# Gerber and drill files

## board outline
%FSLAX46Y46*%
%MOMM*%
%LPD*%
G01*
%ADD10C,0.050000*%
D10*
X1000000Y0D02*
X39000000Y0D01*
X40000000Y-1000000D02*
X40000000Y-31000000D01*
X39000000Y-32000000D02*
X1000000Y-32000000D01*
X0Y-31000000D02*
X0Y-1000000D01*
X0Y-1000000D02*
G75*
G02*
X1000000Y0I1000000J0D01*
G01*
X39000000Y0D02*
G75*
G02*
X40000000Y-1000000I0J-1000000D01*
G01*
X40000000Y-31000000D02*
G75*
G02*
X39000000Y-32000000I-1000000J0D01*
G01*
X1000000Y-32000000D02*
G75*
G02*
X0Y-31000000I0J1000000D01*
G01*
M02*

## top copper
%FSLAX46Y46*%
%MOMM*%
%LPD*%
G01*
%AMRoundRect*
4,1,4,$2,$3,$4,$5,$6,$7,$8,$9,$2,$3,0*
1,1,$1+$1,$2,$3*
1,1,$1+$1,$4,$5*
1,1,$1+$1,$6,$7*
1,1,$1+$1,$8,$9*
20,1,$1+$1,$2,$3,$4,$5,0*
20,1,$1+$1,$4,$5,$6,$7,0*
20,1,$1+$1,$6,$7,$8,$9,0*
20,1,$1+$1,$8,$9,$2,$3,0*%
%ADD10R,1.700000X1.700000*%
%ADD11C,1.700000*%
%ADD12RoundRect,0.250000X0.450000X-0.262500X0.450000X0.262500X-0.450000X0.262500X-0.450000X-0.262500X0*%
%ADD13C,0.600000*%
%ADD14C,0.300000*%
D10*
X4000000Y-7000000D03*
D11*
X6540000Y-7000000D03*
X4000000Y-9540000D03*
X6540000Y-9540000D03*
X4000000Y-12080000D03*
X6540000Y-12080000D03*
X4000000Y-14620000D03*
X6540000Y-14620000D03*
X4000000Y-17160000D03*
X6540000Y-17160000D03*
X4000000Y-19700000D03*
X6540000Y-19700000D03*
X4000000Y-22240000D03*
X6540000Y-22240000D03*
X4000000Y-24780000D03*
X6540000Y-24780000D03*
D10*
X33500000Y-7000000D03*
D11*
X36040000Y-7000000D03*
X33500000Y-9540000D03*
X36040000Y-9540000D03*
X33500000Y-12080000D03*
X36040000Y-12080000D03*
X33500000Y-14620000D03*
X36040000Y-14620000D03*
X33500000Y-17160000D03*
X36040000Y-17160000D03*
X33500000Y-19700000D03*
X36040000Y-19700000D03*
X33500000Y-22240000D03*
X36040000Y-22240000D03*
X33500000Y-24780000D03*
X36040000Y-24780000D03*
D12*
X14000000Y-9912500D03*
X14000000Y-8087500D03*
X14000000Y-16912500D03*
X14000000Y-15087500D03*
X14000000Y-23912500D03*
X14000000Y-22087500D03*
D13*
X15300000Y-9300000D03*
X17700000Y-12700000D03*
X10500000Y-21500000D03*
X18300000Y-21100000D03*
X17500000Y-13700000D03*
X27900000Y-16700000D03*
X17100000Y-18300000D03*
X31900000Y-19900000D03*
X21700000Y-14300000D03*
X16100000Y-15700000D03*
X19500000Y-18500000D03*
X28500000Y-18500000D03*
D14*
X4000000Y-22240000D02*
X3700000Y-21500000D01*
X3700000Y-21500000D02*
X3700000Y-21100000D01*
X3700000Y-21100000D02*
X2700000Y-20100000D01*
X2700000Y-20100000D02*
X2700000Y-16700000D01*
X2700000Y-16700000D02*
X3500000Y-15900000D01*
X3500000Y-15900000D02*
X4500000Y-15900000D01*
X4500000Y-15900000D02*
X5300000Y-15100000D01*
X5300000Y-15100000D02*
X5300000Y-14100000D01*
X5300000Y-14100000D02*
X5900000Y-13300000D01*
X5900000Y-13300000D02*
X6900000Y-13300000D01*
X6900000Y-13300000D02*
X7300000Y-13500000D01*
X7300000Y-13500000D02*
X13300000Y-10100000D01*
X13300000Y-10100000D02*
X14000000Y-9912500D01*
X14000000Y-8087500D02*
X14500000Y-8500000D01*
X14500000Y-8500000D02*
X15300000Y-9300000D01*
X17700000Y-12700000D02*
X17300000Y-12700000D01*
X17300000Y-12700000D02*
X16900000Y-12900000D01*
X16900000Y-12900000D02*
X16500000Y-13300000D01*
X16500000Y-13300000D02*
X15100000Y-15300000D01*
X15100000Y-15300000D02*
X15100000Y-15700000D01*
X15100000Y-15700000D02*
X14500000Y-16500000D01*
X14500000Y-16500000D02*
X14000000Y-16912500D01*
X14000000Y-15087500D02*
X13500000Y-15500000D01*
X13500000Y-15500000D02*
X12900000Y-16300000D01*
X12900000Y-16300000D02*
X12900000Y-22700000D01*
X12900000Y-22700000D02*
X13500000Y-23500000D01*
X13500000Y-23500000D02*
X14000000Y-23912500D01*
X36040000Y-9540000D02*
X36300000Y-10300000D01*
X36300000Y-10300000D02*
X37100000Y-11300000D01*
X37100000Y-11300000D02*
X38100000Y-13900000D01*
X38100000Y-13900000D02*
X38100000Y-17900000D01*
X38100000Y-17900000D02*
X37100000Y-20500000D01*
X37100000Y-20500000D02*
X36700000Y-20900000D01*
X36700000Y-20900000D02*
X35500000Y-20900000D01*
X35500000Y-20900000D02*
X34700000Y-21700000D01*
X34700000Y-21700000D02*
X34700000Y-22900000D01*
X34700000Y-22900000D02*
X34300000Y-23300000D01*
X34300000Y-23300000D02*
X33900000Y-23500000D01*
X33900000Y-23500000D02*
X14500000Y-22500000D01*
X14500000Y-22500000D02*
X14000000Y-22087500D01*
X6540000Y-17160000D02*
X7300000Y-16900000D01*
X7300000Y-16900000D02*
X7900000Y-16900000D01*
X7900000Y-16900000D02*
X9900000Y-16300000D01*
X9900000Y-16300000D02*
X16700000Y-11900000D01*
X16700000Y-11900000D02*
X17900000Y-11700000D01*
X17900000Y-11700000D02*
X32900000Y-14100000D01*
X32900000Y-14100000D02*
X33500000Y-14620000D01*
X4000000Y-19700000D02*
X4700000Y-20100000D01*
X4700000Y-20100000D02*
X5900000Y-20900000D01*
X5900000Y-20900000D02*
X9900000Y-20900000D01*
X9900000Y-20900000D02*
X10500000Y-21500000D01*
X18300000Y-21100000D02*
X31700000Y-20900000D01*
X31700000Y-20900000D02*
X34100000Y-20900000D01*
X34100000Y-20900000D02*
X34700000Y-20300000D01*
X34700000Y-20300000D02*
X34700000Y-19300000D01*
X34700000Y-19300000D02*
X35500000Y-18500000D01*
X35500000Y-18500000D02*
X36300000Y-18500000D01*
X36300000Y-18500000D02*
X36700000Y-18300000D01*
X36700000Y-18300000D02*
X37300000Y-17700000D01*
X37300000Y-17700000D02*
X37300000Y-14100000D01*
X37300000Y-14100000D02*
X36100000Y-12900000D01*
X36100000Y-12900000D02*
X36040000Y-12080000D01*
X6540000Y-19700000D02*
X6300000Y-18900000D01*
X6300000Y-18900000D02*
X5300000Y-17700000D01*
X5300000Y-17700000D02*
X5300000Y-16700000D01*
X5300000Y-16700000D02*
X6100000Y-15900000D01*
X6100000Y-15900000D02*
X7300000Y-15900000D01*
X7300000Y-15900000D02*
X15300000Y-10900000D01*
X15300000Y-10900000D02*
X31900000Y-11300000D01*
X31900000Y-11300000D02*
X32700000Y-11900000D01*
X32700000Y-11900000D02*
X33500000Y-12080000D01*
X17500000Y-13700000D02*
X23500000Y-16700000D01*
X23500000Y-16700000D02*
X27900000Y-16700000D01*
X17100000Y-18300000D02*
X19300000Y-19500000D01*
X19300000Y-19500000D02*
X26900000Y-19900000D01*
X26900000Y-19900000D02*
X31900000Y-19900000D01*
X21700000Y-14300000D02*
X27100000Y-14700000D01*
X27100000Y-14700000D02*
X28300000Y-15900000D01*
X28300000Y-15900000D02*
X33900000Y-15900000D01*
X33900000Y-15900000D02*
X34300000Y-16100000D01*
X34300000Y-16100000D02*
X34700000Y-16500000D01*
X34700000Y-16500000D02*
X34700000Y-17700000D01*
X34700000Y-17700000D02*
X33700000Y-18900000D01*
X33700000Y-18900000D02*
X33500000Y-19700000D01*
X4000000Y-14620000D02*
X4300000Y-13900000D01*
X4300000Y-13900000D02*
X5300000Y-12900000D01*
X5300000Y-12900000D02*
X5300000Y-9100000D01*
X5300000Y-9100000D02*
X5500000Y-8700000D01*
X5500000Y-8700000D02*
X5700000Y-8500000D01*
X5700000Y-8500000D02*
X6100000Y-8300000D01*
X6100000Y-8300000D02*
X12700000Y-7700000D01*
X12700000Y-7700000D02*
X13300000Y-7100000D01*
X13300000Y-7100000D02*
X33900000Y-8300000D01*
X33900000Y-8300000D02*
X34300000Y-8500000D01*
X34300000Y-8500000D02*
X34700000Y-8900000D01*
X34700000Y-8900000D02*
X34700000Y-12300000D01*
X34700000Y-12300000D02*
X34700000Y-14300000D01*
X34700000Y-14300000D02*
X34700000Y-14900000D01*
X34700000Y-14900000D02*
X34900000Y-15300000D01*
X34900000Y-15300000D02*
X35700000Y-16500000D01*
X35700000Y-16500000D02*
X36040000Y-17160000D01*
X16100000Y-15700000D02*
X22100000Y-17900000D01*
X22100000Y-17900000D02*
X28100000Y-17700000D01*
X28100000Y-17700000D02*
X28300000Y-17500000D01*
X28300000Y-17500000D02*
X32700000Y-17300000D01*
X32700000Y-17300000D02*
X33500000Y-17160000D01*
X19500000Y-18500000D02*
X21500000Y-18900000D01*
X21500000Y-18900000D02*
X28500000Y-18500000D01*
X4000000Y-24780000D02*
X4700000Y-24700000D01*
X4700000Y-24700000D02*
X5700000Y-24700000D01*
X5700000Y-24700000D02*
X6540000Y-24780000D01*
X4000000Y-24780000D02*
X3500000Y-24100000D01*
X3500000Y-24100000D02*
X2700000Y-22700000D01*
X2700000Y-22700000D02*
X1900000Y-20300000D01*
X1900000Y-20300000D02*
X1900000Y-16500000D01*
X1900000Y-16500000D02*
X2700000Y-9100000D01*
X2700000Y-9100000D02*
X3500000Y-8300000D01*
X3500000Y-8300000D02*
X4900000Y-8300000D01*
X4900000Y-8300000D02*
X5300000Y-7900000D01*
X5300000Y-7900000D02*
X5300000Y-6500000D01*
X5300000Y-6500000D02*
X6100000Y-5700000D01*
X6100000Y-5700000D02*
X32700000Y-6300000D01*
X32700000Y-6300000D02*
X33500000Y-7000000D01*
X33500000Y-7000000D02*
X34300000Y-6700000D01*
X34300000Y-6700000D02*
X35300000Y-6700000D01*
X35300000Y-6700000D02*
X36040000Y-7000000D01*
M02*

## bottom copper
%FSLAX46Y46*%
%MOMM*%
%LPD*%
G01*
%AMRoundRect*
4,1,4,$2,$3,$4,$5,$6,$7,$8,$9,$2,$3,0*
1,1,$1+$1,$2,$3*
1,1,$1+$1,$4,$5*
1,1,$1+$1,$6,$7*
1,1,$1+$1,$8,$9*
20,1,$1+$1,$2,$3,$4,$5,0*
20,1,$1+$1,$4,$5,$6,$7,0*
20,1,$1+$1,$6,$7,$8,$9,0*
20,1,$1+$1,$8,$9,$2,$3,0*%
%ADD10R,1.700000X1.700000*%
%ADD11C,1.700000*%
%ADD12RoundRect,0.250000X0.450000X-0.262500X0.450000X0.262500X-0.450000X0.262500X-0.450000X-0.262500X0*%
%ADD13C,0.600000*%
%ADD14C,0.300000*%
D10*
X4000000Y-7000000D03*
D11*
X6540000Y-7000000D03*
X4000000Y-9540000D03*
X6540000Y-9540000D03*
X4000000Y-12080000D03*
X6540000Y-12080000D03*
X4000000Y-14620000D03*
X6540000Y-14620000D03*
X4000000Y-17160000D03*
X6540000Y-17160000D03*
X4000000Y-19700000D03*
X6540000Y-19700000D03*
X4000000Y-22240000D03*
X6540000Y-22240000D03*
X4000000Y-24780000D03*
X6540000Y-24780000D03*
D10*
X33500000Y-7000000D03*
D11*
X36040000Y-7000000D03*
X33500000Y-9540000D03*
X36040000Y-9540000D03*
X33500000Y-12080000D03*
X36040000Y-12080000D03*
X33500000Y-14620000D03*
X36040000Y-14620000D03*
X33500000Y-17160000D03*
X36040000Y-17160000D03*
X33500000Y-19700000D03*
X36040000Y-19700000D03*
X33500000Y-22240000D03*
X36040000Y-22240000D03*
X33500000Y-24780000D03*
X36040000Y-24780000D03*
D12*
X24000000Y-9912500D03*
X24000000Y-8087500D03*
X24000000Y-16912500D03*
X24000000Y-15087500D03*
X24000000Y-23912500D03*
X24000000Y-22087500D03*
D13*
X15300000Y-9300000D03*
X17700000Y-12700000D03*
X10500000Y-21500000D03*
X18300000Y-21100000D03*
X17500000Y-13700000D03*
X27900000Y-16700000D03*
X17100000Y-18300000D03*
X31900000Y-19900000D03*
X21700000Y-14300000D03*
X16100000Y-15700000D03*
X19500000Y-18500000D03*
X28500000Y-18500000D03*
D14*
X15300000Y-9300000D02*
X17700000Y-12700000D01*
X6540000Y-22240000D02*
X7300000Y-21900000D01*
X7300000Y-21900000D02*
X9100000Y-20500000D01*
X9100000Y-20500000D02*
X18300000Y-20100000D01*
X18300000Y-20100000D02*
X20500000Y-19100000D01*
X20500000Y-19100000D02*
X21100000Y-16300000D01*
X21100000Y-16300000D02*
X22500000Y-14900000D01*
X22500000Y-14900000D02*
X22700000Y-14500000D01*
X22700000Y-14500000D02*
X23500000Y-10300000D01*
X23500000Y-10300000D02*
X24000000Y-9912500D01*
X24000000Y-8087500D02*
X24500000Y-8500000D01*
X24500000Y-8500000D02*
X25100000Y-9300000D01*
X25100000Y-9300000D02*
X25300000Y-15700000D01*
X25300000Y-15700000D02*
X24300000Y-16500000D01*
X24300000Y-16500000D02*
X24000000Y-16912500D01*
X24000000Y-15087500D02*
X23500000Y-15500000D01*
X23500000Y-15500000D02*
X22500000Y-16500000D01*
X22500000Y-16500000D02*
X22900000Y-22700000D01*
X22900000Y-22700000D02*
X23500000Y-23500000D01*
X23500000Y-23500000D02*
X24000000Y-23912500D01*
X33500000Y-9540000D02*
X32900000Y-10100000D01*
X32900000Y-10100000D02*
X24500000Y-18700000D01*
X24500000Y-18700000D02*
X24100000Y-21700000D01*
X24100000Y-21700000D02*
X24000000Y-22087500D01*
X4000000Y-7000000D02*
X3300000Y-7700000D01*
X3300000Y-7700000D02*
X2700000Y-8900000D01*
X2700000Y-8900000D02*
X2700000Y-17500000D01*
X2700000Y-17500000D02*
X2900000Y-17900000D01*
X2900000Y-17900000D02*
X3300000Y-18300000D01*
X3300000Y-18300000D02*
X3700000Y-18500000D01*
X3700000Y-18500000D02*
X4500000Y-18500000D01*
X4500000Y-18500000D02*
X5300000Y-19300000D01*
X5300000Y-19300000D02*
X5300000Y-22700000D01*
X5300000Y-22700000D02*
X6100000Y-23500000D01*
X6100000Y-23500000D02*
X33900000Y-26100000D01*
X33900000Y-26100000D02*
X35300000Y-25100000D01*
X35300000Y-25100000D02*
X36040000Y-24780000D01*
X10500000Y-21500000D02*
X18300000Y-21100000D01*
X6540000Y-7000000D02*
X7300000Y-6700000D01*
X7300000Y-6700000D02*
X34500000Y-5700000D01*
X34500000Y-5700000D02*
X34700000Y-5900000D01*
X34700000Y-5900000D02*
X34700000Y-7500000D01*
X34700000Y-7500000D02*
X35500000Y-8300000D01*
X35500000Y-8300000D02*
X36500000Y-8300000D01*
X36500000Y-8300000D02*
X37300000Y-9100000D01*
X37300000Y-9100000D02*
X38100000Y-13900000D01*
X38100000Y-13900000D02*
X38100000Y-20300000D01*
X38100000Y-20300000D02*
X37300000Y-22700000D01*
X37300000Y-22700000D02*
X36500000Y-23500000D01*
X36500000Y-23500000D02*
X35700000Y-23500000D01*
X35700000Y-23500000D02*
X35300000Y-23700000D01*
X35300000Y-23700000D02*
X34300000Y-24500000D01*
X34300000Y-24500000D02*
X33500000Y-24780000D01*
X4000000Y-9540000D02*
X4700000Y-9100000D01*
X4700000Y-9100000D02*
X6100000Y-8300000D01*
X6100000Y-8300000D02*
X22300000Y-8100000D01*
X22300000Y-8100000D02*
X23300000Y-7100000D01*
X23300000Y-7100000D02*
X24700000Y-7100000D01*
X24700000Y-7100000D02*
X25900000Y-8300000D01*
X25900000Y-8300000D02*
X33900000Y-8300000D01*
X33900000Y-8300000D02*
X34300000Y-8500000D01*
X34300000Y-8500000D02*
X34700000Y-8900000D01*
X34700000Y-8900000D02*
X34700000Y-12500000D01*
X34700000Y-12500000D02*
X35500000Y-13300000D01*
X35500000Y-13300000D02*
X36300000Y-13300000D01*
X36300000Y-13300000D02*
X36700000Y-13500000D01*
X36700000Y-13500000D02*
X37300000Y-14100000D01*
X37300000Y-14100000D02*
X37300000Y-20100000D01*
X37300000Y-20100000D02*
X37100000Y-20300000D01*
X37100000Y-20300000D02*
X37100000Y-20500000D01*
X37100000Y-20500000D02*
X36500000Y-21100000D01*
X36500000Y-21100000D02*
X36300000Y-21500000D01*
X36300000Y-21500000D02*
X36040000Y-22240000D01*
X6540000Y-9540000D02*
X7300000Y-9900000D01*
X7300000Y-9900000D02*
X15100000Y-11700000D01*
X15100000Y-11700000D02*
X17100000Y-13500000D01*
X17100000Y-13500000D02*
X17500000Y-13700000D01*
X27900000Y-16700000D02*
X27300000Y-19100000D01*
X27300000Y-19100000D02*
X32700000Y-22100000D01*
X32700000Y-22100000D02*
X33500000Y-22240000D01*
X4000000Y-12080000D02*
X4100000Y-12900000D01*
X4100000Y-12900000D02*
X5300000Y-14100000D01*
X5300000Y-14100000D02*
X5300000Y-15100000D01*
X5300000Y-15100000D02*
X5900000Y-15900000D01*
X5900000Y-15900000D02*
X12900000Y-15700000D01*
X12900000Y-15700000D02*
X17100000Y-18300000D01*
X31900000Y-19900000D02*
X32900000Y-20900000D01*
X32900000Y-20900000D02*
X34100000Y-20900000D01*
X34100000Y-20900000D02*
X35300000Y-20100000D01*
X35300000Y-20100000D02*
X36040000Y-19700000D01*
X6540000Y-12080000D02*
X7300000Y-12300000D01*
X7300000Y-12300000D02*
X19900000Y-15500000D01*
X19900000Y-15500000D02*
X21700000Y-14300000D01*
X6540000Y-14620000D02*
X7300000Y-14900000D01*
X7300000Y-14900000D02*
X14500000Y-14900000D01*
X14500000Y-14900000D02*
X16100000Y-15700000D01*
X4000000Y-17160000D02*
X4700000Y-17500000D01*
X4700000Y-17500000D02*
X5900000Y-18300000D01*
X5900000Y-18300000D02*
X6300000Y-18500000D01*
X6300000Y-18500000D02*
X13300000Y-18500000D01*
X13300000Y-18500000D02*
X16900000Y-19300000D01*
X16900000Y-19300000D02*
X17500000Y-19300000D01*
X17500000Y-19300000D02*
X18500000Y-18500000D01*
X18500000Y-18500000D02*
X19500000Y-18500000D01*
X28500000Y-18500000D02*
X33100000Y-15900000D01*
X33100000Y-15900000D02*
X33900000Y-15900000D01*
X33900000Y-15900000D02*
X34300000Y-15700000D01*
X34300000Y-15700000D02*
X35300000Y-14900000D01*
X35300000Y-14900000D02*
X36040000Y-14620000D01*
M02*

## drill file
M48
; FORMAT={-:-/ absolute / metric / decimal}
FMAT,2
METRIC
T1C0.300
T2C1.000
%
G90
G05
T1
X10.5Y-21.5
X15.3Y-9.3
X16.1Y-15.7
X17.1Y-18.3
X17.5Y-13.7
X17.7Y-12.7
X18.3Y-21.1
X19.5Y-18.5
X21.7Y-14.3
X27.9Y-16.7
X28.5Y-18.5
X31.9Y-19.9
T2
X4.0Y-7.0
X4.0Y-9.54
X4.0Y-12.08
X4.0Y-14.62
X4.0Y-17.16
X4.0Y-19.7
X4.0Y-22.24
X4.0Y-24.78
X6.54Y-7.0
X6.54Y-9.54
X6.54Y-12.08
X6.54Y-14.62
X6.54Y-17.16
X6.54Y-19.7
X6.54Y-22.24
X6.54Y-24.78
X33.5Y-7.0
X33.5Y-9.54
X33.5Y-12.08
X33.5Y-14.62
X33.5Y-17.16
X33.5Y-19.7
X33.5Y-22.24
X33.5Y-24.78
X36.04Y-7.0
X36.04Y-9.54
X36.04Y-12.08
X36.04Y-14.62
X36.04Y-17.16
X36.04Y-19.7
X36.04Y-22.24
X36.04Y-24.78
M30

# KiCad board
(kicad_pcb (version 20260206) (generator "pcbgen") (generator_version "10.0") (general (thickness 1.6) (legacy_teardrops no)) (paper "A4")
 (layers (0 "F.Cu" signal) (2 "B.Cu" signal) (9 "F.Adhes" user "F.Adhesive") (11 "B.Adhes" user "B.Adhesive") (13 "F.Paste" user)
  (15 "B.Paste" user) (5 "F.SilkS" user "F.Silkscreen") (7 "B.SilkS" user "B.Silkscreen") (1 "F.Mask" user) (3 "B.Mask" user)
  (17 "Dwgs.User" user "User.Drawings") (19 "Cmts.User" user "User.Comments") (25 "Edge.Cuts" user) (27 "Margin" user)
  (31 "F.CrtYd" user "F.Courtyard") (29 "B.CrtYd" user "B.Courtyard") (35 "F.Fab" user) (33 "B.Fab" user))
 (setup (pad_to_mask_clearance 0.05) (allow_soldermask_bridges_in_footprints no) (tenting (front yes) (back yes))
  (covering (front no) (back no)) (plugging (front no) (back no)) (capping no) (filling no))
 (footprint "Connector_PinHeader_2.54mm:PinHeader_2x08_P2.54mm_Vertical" (layer "F.Cu") (at 4 7)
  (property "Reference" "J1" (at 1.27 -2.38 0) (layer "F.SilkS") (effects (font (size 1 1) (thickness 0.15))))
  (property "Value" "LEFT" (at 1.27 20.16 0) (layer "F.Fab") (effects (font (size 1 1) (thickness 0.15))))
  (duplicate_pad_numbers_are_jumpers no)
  (pad "1" thru_hole rect (at 0 0) (size 1.7 1.7) (drill 1) (layers "*.Cu" "*.Mask") (remove_unused_layers no) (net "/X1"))
  (pad "2" thru_hole circle (at 2.54 0) (size 1.7 1.7) (drill 1) (layers "*.Cu" "*.Mask") (remove_unused_layers no) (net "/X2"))
  (pad "3" thru_hole circle (at 0 2.54) (size 1.7 1.7) (drill 1) (layers "*.Cu" "*.Mask") (remove_unused_layers no) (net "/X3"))
  (pad "4" thru_hole circle (at 2.54 2.54) (size 1.7 1.7) (drill 1) (layers "*.Cu" "*.Mask") (remove_unused_layers no) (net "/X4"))
  (pad "5" thru_hole circle (at 0 5.08) (size 1.7 1.7) (drill 1) (layers "*.Cu" "*.Mask") (remove_unused_layers no) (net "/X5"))
  (pad "6" thru_hole circle (at 2.54 5.08) (size 1.7 1.7) (drill 1) (layers "*.Cu" "*.Mask") (remove_unused_layers no) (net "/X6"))
  (pad "7" thru_hole circle (at 0 7.62) (size 1.7 1.7) (drill 1) (layers "*.Cu" "*.Mask") (remove_unused_layers no) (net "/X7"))
  (pad "8" thru_hole circle (at 2.54 7.62) (size 1.7 1.7) (drill 1) (layers "*.Cu" "*.Mask") (remove_unused_layers no) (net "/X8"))
  (pad "9" thru_hole circle (at 0 10.16) (size 1.7 1.7) (drill 1) (layers "*.Cu" "*.Mask") (remove_unused_layers no) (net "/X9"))
  (pad "10" thru_hole circle (at 2.54 10.16) (size 1.7 1.7) (drill 1) (layers "*.Cu" "*.Mask") (remove_unused_layers no) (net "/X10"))
  (pad "11" thru_hole circle (at 0 12.7) (size 1.7 1.7) (drill 1) (layers "*.Cu" "*.Mask") (remove_unused_layers no) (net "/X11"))
  (pad "12" thru_hole circle (at 2.54 12.7) (size 1.7 1.7) (drill 1) (layers "*.Cu" "*.Mask") (remove_unused_layers no) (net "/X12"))
  (pad "13" thru_hole circle (at 0 15.24) (size 1.7 1.7) (drill 1) (layers "*.Cu" "*.Mask") (remove_unused_layers no) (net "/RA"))
  (pad "14" thru_hole circle (at 2.54 15.24) (size 1.7 1.7) (drill 1) (layers "*.Cu" "*.Mask") (remove_unused_layers no) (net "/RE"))
  (pad "15" thru_hole circle (at 0 17.78) (size 1.7 1.7) (drill 1) (layers "*.Cu" "*.Mask") (remove_unused_layers no) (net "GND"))
  (pad "16" thru_hole circle (at 2.54 17.78) (size 1.7 1.7) (drill 1) (layers "*.Cu" "*.Mask") (remove_unused_layers no) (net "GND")))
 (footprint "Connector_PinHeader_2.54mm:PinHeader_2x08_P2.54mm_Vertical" (layer "F.Cu") (at 33.5 7)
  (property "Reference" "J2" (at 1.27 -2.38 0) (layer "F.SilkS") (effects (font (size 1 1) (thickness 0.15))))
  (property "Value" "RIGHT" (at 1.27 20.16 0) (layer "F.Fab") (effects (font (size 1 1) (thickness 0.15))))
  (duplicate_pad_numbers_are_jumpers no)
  (pad "1" thru_hole rect (at 0 0) (size 1.7 1.7) (drill 1) (layers "*.Cu" "*.Mask") (remove_unused_layers no) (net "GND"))
  (pad "2" thru_hole circle (at 2.54 0) (size 1.7 1.7) (drill 1) (layers "*.Cu" "*.Mask") (remove_unused_layers no) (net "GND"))
  (pad "3" thru_hole circle (at 0 2.54) (size 1.7 1.7) (drill 1) (layers "*.Cu" "*.Mask") (remove_unused_layers no) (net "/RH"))
  (pad "4" thru_hole circle (at 2.54 2.54) (size 1.7 1.7) (drill 1) (layers "*.Cu" "*.Mask") (remove_unused_layers no) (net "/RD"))
  (pad "5" thru_hole circle (at 0 5.08) (size 1.7 1.7) (drill 1) (layers "*.Cu" "*.Mask") (remove_unused_layers no) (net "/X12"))
  (pad "6" thru_hole circle (at 2.54 5.08) (size 1.7 1.7) (drill 1) (layers "*.Cu" "*.Mask") (remove_unused_layers no) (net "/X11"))
  (pad "7" thru_hole circle (at 0 7.62) (size 1.7 1.7) (drill 1) (layers "*.Cu" "*.Mask") (remove_unused_layers no) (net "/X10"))
  (pad "8" thru_hole circle (at 2.54 7.62) (size 1.7 1.7) (drill 1) (layers "*.Cu" "*.Mask") (remove_unused_layers no) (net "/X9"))
  (pad "9" thru_hole circle (at 0 10.16) (size 1.7 1.7) (drill 1) (layers "*.Cu" "*.Mask") (remove_unused_layers no) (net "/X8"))
  (pad "10" thru_hole circle (at 2.54 10.16) (size 1.7 1.7) (drill 1) (layers "*.Cu" "*.Mask") (remove_unused_layers no) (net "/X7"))
  (pad "11" thru_hole circle (at 0 12.7) (size 1.7 1.7) (drill 1) (layers "*.Cu" "*.Mask") (remove_unused_layers no) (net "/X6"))
  (pad "12" thru_hole circle (at 2.54 12.7) (size 1.7 1.7) (drill 1) (layers "*.Cu" "*.Mask") (remove_unused_layers no) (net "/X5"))
  (pad "13" thru_hole circle (at 0 15.24) (size 1.7 1.7) (drill 1) (layers "*.Cu" "*.Mask") (remove_unused_layers no) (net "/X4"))
  (pad "14" thru_hole circle (at 2.54 15.24) (size 1.7 1.7) (drill 1) (layers "*.Cu" "*.Mask") (remove_unused_layers no) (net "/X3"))
  (pad "15" thru_hole circle (at 0 17.78) (size 1.7 1.7) (drill 1) (layers "*.Cu" "*.Mask") (remove_unused_layers no) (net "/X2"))
  (pad "16" thru_hole circle (at 2.54 17.78) (size 1.7 1.7) (drill 1) (layers "*.Cu" "*.Mask") (remove_unused_layers no) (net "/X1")))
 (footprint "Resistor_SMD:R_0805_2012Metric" (layer "F.Cu") (at 14 9 90)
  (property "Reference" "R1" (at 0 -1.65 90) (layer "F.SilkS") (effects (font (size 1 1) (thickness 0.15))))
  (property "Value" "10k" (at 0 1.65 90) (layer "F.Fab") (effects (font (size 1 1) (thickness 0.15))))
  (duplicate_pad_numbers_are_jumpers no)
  (pad "1" smd roundrect (at -0.9125 0 90) (size 1.025 1.4) (layers "F.Cu" "F.Mask" "F.Paste") (roundrect_rratio 0.243902) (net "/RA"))
  (pad "2" smd roundrect (at 0.9125 0 90) (size 1.025 1.4) (layers "F.Cu" "F.Mask" "F.Paste") (roundrect_rratio 0.243902) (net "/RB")))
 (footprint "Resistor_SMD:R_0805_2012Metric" (layer "F.Cu") (at 14 16 90)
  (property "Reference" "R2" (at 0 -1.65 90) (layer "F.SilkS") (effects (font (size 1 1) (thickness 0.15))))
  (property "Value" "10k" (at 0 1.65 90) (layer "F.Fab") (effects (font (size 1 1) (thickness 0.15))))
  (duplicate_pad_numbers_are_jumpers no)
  (pad "1" smd roundrect (at -0.9125 0 90) (size 1.025 1.4) (layers "F.Cu" "F.Mask" "F.Paste") (roundrect_rratio 0.243902) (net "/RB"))
  (pad "2" smd roundrect (at 0.9125 0 90) (size 1.025 1.4) (layers "F.Cu" "F.Mask" "F.Paste") (roundrect_rratio 0.243902) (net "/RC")))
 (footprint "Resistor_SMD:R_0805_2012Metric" (layer "F.Cu") (at 14 23 90)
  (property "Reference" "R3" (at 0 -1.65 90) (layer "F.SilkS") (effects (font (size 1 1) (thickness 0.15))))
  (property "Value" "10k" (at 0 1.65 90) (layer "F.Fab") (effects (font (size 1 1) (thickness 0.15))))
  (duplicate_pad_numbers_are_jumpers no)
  (pad "1" smd roundrect (at -0.9125 0 90) (size 1.025 1.4) (layers "F.Cu" "F.Mask" "F.Paste") (roundrect_rratio 0.243902) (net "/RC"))
  (pad "2" smd roundrect (at 0.9125 0 90) (size 1.025 1.4) (layers "F.Cu" "F.Mask" "F.Paste") (roundrect_rratio 0.243902) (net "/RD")))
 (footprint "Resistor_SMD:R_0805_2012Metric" (layer "B.Cu") (at 24 9 90)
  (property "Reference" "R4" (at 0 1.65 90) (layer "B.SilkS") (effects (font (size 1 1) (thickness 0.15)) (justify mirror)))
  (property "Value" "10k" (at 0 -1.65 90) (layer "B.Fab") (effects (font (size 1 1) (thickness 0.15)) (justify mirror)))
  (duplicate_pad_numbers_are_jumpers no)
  (pad "1" smd roundrect (at -0.9125 0 90) (size 1.025 1.4) (layers "B.Cu" "B.Mask" "B.Paste") (roundrect_rratio 0.243902) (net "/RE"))
  (pad "2" smd roundrect (at 0.9125 0 90) (size 1.025 1.4) (layers "B.Cu" "B.Mask" "B.Paste") (roundrect_rratio 0.243902) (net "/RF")))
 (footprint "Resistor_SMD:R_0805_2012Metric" (layer "B.Cu") (at 24 16 90)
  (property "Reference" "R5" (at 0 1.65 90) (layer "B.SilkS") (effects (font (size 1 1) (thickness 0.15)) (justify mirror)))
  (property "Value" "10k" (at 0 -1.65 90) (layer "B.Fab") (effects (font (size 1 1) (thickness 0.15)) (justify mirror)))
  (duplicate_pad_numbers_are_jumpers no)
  (pad "1" smd roundrect (at -0.9125 0 90) (size 1.025 1.4) (layers "B.Cu" "B.Mask" "B.Paste") (roundrect_rratio 0.243902) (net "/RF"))
  (pad "2" smd roundrect (at 0.9125 0 90) (size 1.025 1.4) (layers "B.Cu" "B.Mask" "B.Paste") (roundrect_rratio 0.243902) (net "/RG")))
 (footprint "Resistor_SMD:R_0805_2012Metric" (layer "B.Cu") (at 24 23 90)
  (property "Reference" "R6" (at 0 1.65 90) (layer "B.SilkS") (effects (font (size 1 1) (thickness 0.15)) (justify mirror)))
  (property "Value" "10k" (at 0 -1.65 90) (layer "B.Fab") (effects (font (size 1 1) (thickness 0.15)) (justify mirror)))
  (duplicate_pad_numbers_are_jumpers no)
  (pad "1" smd roundrect (at -0.9125 0 90) (size 1.025 1.4) (layers "B.Cu" "B.Mask" "B.Paste") (roundrect_rratio 0.243902) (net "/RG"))
  (pad "2" smd roundrect (at 0.9125 0 90) (size 1.025 1.4) (layers "B.Cu" "B.Mask" "B.Paste") (roundrect_rratio 0.243902) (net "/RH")))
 (gr_line (start 1 0) (end 39 0) (stroke (width 0.05) (type default)) (layer "Edge.Cuts"))
 (gr_line (start 40 1) (end 40 31) (stroke (width 0.05) (type default)) (layer "Edge.Cuts"))
 (gr_line (start 39 32) (end 1 32) (stroke (width 0.05) (type default)) (layer "Edge.Cuts"))
 (gr_line (start 0 31) (end 0 1) (stroke (width 0.05) (type default)) (layer "Edge.Cuts"))
 (gr_arc (start 0 1) (mid 0.292893 0.292893) (end 1 0) (stroke (width 0.05) (type default)) (layer "Edge.Cuts"))
 (gr_arc (start 39 0) (mid 39.707107 0.292893) (end 40 1) (stroke (width 0.05) (type default)) (layer "Edge.Cuts"))
 (gr_arc (start 40 31) (mid 39.707107 31.707107) (end 39 32) (stroke (width 0.05) (type default)) (layer "Edge.Cuts"))
 (gr_arc (start 1 32) (mid 0.292893 31.707107) (end 0 31) (stroke (width 0.05) (type default)) (layer "Edge.Cuts"))
 (segment (start 4 22.24) (end 3.7 21.5) (width 0.3) (layer "F.Cu") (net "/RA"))
 (segment (start 3.7 21.5) (end 3.7 21.1) (width 0.3) (layer "F.Cu") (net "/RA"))
 (segment (start 3.7 21.1) (end 2.7 20.1) (width 0.3) (layer "F.Cu") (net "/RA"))
 (segment (start 2.7 20.1) (end 2.7 16.7) (width 0.3) (layer "F.Cu") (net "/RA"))
 (segment (start 2.7 16.7) (end 3.5 15.9) (width 0.3) (layer "F.Cu") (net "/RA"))
 (segment (start 3.5 15.9) (end 4.5 15.9) (width 0.3) (layer "F.Cu") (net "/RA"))
 (segment (start 4.5 15.9) (end 5.3 15.1) (width 0.3) (layer "F.Cu") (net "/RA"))
 (segment (start 5.3 15.1) (end 5.3 14.1) (width 0.3) (layer "F.Cu") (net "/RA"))
 (segment (start 5.3 14.1) (end 5.9 13.3) (width 0.3) (layer "F.Cu") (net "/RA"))
 (segment (start 5.9 13.3) (end 6.9 13.3) (width 0.3) (layer "F.Cu") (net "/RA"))
 (segment (start 6.9 13.3) (end 7.3 13.5) (width 0.3) (layer "F.Cu") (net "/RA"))
 (segment (start 7.3 13.5) (end 13.3 10.1) (width 0.3) (layer "F.Cu") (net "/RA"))
 (segment (start 13.3 10.1) (end 14 9.9125) (width 0.3) (layer "F.Cu") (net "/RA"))
 (segment (start 14 8.0875) (end 14.5 8.5) (width 0.3) (layer "F.Cu") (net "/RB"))
 (segment (start 14.5 8.5) (end 15.3 9.3) (width 0.3) (layer "F.Cu") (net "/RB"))
 (segment (start 15.3 9.3) (end 17.7 12.7) (width 0.3) (layer "B.Cu") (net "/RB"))
 (segment (start 17.7 12.7) (end 17.3 12.7) (width 0.3) (layer "F.Cu") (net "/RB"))
 (segment (start 17.3 12.7) (end 16.9 12.9) (width 0.3) (layer "F.Cu") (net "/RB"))
 (segment (start 16.9 12.9) (end 16.5 13.3) (width 0.3) (layer "F.Cu") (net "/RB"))
 (segment (start 16.5 13.3) (end 15.1 15.3) (width 0.3) (layer "F.Cu") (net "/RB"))
 (segment (start 15.1 15.3) (end 15.1 15.7) (width 0.3) (layer "F.Cu") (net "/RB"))
 (segment (start 15.1 15.7) (end 14.5 16.5) (width 0.3) (layer "F.Cu") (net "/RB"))
 (segment (start 14.5 16.5) (end 14 16.9125) (width 0.3) (layer "F.Cu") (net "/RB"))
 (segment (start 14 15.0875) (end 13.5 15.5) (width 0.3) (layer "F.Cu") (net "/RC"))
 (segment (start 13.5 15.5) (end 12.9 16.3) (width 0.3) (layer "F.Cu") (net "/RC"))
 (segment (start 12.9 16.3) (end 12.9 22.7) (width 0.3) (layer "F.Cu") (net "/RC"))
 (segment (start 12.9 22.7) (end 13.5 23.5) (width 0.3) (layer "F.Cu") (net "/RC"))
 (segment (start 13.5 23.5) (end 14 23.9125) (width 0.3) (layer "F.Cu") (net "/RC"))
 (segment (start 36.04 9.54) (end 36.3 10.3) (width 0.3) (layer "F.Cu") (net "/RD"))
 (segment (start 36.3 10.3) (end 37.1 11.3) (width 0.3) (layer "F.Cu") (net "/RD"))
 (segment (start 37.1 11.3) (end 38.1 13.9) (width 0.3) (layer "F.Cu") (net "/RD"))
 (segment (start 38.1 13.9) (end 38.1 17.9) (width 0.3) (layer "F.Cu") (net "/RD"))
 (segment (start 38.1 17.9) (end 37.1 20.5) (width 0.3) (layer "F.Cu") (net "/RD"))
 (segment (start 37.1 20.5) (end 36.7 20.9) (width 0.3) (layer "F.Cu") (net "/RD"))
 (segment (start 36.7 20.9) (end 35.5 20.9) (width 0.3) (layer "F.Cu") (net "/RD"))
 (segment (start 35.5 20.9) (end 34.7 21.7) (width 0.3) (layer "F.Cu") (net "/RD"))
 (segment (start 34.7 21.7) (end 34.7 22.9) (width 0.3) (layer "F.Cu") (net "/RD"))
 (segment (start 34.7 22.9) (end 34.3 23.3) (width 0.3) (layer "F.Cu") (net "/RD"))
 (segment (start 34.3 23.3) (end 33.9 23.5) (width 0.3) (layer "F.Cu") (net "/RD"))
 (segment (start 33.9 23.5) (end 14.5 22.5) (width 0.3) (layer "F.Cu") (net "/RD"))
 (segment (start 14.5 22.5) (end 14 22.0875) (width 0.3) (layer "F.Cu") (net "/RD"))
 (segment (start 6.54 22.24) (end 7.3 21.9) (width 0.3) (layer "B.Cu") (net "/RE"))
 (segment (start 7.3 21.9) (end 9.1 20.5) (width 0.3) (layer "B.Cu") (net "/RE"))
 (segment (start 9.1 20.5) (end 18.3 20.1) (width 0.3) (layer "B.Cu") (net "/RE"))
 (segment (start 18.3 20.1) (end 20.5 19.1) (width 0.3) (layer "B.Cu") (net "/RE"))
 (segment (start 20.5 19.1) (end 21.1 16.3) (width 0.3) (layer "B.Cu") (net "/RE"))
 (segment (start 21.1 16.3) (end 22.5 14.9) (width 0.3) (layer "B.Cu") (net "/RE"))
 (segment (start 22.5 14.9) (end 22.7 14.5) (width 0.3) (layer "B.Cu") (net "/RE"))
 (segment (start 22.7 14.5) (end 23.5 10.3) (width 0.3) (layer "B.Cu") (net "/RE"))
 (segment (start 23.5 10.3) (end 24 9.9125) (width 0.3) (layer "B.Cu") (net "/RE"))
 (segment (start 24 8.0875) (end 24.5 8.5) (width 0.3) (layer "B.Cu") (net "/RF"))
 (segment (start 24.5 8.5) (end 25.1 9.3) (width 0.3) (layer "B.Cu") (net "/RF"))
 (segment (start 25.1 9.3) (end 25.3 15.7) (width 0.3) (layer "B.Cu") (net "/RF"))
 (segment (start 25.3 15.7) (end 24.3 16.5) (width 0.3) (layer "B.Cu") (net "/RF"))
 (segment (start 24.3 16.5) (end 24 16.9125) (width 0.3) (layer "B.Cu") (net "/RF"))
 (segment (start 24 15.0875) (end 23.5 15.5) (width 0.3) (layer "B.Cu") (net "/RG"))
 (segment (start 23.5 15.5) (end 22.5 16.5) (width 0.3) (layer "B.Cu") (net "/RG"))
 (segment (start 22.5 16.5) (end 22.9 22.7) (width 0.3) (layer "B.Cu") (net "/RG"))
 (segment (start 22.9 22.7) (end 23.5 23.5) (width 0.3) (layer "B.Cu") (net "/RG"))
 (segment (start 23.5 23.5) (end 24 23.9125) (width 0.3) (layer "B.Cu") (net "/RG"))
 (segment (start 33.5 9.54) (end 32.9 10.1) (width 0.3) (layer "B.Cu") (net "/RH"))
 (segment (start 32.9 10.1) (end 24.5 18.7) (width 0.3) (layer "B.Cu") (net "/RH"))
 (segment (start 24.5 18.7) (end 24.1 21.7) (width 0.3) (layer "B.Cu") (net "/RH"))
 (segment (start 24.1 21.7) (end 24 22.0875) (width 0.3) (layer "B.Cu") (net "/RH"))
 (segment (start 4 7) (end 3.3 7.7) (width 0.3) (layer "B.Cu") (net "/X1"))
 (segment (start 3.3 7.7) (end 2.7 8.9) (width 0.3) (layer "B.Cu") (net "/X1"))
 (segment (start 2.7 8.9) (end 2.7 17.5) (width 0.3) (layer "B.Cu") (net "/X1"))
 (segment (start 2.7 17.5) (end 2.9 17.9) (width 0.3) (layer "B.Cu") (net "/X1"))
 (segment (start 2.9 17.9) (end 3.3 18.3) (width 0.3) (layer "B.Cu") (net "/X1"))
 (segment (start 3.3 18.3) (end 3.7 18.5) (width 0.3) (layer "B.Cu") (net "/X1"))
 (segment (start 3.7 18.5) (end 4.5 18.5) (width 0.3) (layer "B.Cu") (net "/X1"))
 (segment (start 4.5 18.5) (end 5.3 19.3) (width 0.3) (layer "B.Cu") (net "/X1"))
 (segment (start 5.3 19.3) (end 5.3 22.7) (width 0.3) (layer "B.Cu") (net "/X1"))
 (segment (start 5.3 22.7) (end 6.1 23.5) (width 0.3) (layer "B.Cu") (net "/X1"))
 (segment (start 6.1 23.5) (end 33.9 26.1) (width 0.3) (layer "B.Cu") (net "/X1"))
 (segment (start 33.9 26.1) (end 35.3 25.1) (width 0.3) (layer "B.Cu") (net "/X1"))
 (segment (start 35.3 25.1) (end 36.04 24.78) (width 0.3) (layer "B.Cu") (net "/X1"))
 (segment (start 6.54 17.16) (end 7.3 16.9) (width 0.3) (layer "F.Cu") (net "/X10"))
 (segment (start 7.3 16.9) (end 7.9 16.9) (width 0.3) (layer "F.Cu") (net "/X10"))
 (segment (start 7.9 16.9) (end 9.9 16.3) (width 0.3) (layer "F.Cu") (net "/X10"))
 (segment (start 9.9 16.3) (end 16.7 11.9) (width 0.3) (layer "F.Cu") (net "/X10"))
 (segment (start 16.7 11.9) (end 17.9 11.7) (width 0.3) (layer "F.Cu") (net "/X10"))
 (segment (start 17.9 11.7) (end 32.9 14.1) (width 0.3) (layer "F.Cu") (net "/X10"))
 (segment (start 32.9 14.1) (end 33.5 14.62) (width 0.3) (layer "F.Cu") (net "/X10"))
 (segment (start 4 19.7) (end 4.7 20.1) (width 0.3) (layer "F.Cu") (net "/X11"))
 (segment (start 4.7 20.1) (end 5.9 20.9) (width 0.3) (layer "F.Cu") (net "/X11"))
 (segment (start 5.9 20.9) (end 9.9 20.9) (width 0.3) (layer "F.Cu") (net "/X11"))
 (segment (start 9.9 20.9) (end 10.5 21.5) (width 0.3) (layer "F.Cu") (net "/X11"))
 (segment (start 10.5 21.5) (end 18.3 21.1) (width 0.3) (layer "B.Cu") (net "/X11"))
 (segment (start 18.3 21.1) (end 31.7 20.9) (width 0.3) (layer "F.Cu") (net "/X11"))
 (segment (start 31.7 20.9) (end 34.1 20.9) (width 0.3) (layer "F.Cu") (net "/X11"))
 (segment (start 34.1 20.9) (end 34.7 20.3) (width 0.3) (layer "F.Cu") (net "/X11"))
 (segment (start 34.7 20.3) (end 34.7 19.3) (width 0.3) (layer "F.Cu") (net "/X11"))
 (segment (start 34.7 19.3) (end 35.5 18.5) (width 0.3) (layer "F.Cu") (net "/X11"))
 (segment (start 35.5 18.5) (end 36.3 18.5) (width 0.3) (layer "F.Cu") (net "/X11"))
 (segment (start 36.3 18.5) (end 36.7 18.3) (width 0.3) (layer "F.Cu") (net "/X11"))
 (segment (start 36.7 18.3) (end 37.3 17.7) (width 0.3) (layer "F.Cu") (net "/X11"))
 (segment (start 37.3 17.7) (end 37.3 14.1) (width 0.3) (layer "F.Cu") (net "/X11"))
 (segment (start 37.3 14.1) (end 36.1 12.9) (width 0.3) (layer "F.Cu") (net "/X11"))
 (segment (start 36.1 12.9) (end 36.04 12.08) (width 0.3) (layer "F.Cu") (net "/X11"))
 (segment (start 6.54 19.7) (end 6.3 18.9) (width 0.3) (layer "F.Cu") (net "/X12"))
 (segment (start 6.3 18.9) (end 5.3 17.7) (width 0.3) (layer "F.Cu") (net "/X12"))
 (segment (start 5.3 17.7) (end 5.3 16.7) (width 0.3) (layer "F.Cu") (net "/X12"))
 (segment (start 5.3 16.7) (end 6.1 15.9) (width 0.3) (layer "F.Cu") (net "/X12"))
 (segment (start 6.1 15.9) (end 7.3 15.9) (width 0.3) (layer "F.Cu") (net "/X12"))
 (segment (start 7.3 15.9) (end 15.3 10.9) (width 0.3) (layer "F.Cu") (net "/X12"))
 (segment (start 15.3 10.9) (end 31.9 11.3) (width 0.3) (layer "F.Cu") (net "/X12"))
 (segment (start 31.9 11.3) (end 32.7 11.9) (width 0.3) (layer "F.Cu") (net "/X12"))
 (segment (start 32.7 11.9) (end 33.5 12.08) (width 0.3) (layer "F.Cu") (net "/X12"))
 (segment (start 6.54 7) (end 7.3 6.7) (width 0.3) (layer "B.Cu") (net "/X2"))
 (segment (start 7.3 6.7) (end 34.5 5.7) (width 0.3) (layer "B.Cu") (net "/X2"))
 (segment (start 34.5 5.7) (end 34.7 5.9) (width 0.3) (layer "B.Cu") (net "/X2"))
 (segment (start 34.7 5.9) (end 34.7 7.5) (width 0.3) (layer "B.Cu") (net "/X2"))
 (segment (start 34.7 7.5) (end 35.5 8.3) (width 0.3) (layer "B.Cu") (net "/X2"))
 (segment (start 35.5 8.3) (end 36.5 8.3) (width 0.3) (layer "B.Cu") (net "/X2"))
 (segment (start 36.5 8.3) (end 37.3 9.1) (width 0.3) (layer "B.Cu") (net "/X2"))
 (segment (start 37.3 9.1) (end 38.1 13.9) (width 0.3) (layer "B.Cu") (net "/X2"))
 (segment (start 38.1 13.9) (end 38.1 20.3) (width 0.3) (layer "B.Cu") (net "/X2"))
 (segment (start 38.1 20.3) (end 37.3 22.7) (width 0.3) (layer "B.Cu") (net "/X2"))
 (segment (start 37.3 22.7) (end 36.5 23.5) (width 0.3) (layer "B.Cu") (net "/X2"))
 (segment (start 36.5 23.5) (end 35.7 23.5) (width 0.3) (layer "B.Cu") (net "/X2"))
 (segment (start 35.7 23.5) (end 35.3 23.7) (width 0.3) (layer "B.Cu") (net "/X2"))
 (segment (start 35.3 23.7) (end 34.3 24.5) (width 0.3) (layer "B.Cu") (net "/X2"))
 (segment (start 34.3 24.5) (end 33.5 24.78) (width 0.3) (layer "B.Cu") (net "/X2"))
 (segment (start 4 9.54) (end 4.7 9.1) (width 0.3) (layer "B.Cu") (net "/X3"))
 (segment (start 4.7 9.1) (end 6.1 8.3) (width 0.3) (layer "B.Cu") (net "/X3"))
 (segment (start 6.1 8.3) (end 22.3 8.1) (width 0.3) (layer "B.Cu") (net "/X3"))
 (segment (start 22.3 8.1) (end 23.3 7.1) (width 0.3) (layer "B.Cu") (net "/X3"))
 (segment (start 23.3 7.1) (end 24.7 7.1) (width 0.3) (layer "B.Cu") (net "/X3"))
 (segment (start 24.7 7.1) (end 25.9 8.3) (width 0.3) (layer "B.Cu") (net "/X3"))
 (segment (start 25.9 8.3) (end 33.9 8.3) (width 0.3) (layer "B.Cu") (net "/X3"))
 (segment (start 33.9 8.3) (end 34.3 8.5) (width 0.3) (layer "B.Cu") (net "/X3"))
 (segment (start 34.3 8.5) (end 34.7 8.9) (width 0.3) (layer "B.Cu") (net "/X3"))
 (segment (start 34.7 8.9) (end 34.7 12.5) (width 0.3) (layer "B.Cu") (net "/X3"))
 (segment (start 34.7 12.5) (end 35.5 13.3) (width 0.3) (layer "B.Cu") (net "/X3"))
 (segment (start 35.5 13.3) (end 36.3 13.3) (width 0.3) (layer "B.Cu") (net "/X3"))
 (segment (start 36.3 13.3) (end 36.7 13.5) (width 0.3) (layer "B.Cu") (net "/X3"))
 (segment (start 36.7 13.5) (end 37.3 14.1) (width 0.3) (layer "B.Cu") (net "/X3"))
 (segment (start 37.3 14.1) (end 37.3 20.1) (width 0.3) (layer "B.Cu") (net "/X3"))
 (segment (start 37.3 20.1) (end 37.1 20.3) (width 0.3) (layer "B.Cu") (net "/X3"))
 (segment (start 37.1 20.3) (end 37.1 20.5) (width 0.3) (layer "B.Cu") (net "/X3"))
 (segment (start 37.1 20.5) (end 36.5 21.1) (width 0.3) (layer "B.Cu") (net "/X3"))
 (segment (start 36.5 21.1) (end 36.3 21.5) (width 0.3) (layer "B.Cu") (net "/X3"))
 (segment (start 36.3 21.5) (end 36.04 22.24) (width 0.3) (layer "B.Cu") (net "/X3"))
 (segment (start 6.54 9.54) (end 7.3 9.9) (width 0.3) (layer "B.Cu") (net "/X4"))
 (segment (start 7.3 9.9) (end 15.1 11.7) (width 0.3) (layer "B.Cu") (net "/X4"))
 (segment (start 15.1 11.7) (end 17.1 13.5) (width 0.3) (layer "B.Cu") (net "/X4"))
 (segment (start 17.1 13.5) (end 17.5 13.7) (width 0.3) (layer "B.Cu") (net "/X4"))
 (segment (start 17.5 13.7) (end 23.5 16.7) (width 0.3) (layer "F.Cu") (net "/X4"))
 (segment (start 23.5 16.7) (end 27.9 16.7) (width 0.3) (layer "F.Cu") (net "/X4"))
 (segment (start 27.9 16.7) (end 27.3 19.1) (width 0.3) (layer "B.Cu") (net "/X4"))
 (segment (start 27.3 19.1) (end 32.7 22.1) (width 0.3) (layer "B.Cu") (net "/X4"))
 (segment (start 32.7 22.1) (end 33.5 22.24) (width 0.3) (layer "B.Cu") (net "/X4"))
 (segment (start 4 12.08) (end 4.1 12.9) (width 0.3) (layer "B.Cu") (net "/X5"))
 (segment (start 4.1 12.9) (end 5.3 14.1) (width 0.3) (layer "B.Cu") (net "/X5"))
 (segment (start 5.3 14.1) (end 5.3 15.1) (width 0.3) (layer "B.Cu") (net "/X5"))
 (segment (start 5.3 15.1) (end 5.9 15.9) (width 0.3) (layer "B.Cu") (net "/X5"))
 (segment (start 5.9 15.9) (end 12.9 15.7) (width 0.3) (layer "B.Cu") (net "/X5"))
 (segment (start 12.9 15.7) (end 17.1 18.3) (width 0.3) (layer "B.Cu") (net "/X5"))
 (segment (start 17.1 18.3) (end 19.3 19.5) (width 0.3) (layer "F.Cu") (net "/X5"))
 (segment (start 19.3 19.5) (end 26.9 19.9) (width 0.3) (layer "F.Cu") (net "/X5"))
 (segment (start 26.9 19.9) (end 31.9 19.9) (width 0.3) (layer "F.Cu") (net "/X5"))
 (segment (start 31.9 19.9) (end 32.9 20.9) (width 0.3) (layer "B.Cu") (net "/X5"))
 (segment (start 32.9 20.9) (end 34.1 20.9) (width 0.3) (layer "B.Cu") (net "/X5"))
 (segment (start 34.1 20.9) (end 35.3 20.1) (width 0.3) (layer "B.Cu") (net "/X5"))
 (segment (start 35.3 20.1) (end 36.04 19.7) (width 0.3) (layer "B.Cu") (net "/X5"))
 (segment (start 6.54 12.08) (end 7.3 12.3) (width 0.3) (layer "B.Cu") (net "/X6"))
 (segment (start 7.3 12.3) (end 19.9 15.5) (width 0.3) (layer "B.Cu") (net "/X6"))
 (segment (start 19.9 15.5) (end 21.7 14.3) (width 0.3) (layer "B.Cu") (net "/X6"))
 (segment (start 21.7 14.3) (end 27.1 14.7) (width 0.3) (layer "F.Cu") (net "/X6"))
 (segment (start 27.1 14.7) (end 28.3 15.9) (width 0.3) (layer "F.Cu") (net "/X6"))
 (segment (start 28.3 15.9) (end 33.9 15.9) (width 0.3) (layer "F.Cu") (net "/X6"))
 (segment (start 33.9 15.9) (end 34.3 16.1) (width 0.3) (layer "F.Cu") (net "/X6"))
 (segment (start 34.3 16.1) (end 34.7 16.5) (width 0.3) (layer "F.Cu") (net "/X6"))
 (segment (start 34.7 16.5) (end 34.7 17.7) (width 0.3) (layer "F.Cu") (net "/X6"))
 (segment (start 34.7 17.7) (end 33.7 18.9) (width 0.3) (layer "F.Cu") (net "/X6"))
 (segment (start 33.7 18.9) (end 33.5 19.7) (width 0.3) (layer "F.Cu") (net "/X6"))
 (segment (start 4 14.62) (end 4.3 13.9) (width 0.3) (layer "F.Cu") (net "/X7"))
 (segment (start 4.3 13.9) (end 5.3 12.9) (width 0.3) (layer "F.Cu") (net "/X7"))
 (segment (start 5.3 12.9) (end 5.3 9.1) (width 0.3) (layer "F.Cu") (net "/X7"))
 (segment (start 5.3 9.1) (end 5.5 8.7) (width 0.3) (layer "F.Cu") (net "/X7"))
 (segment (start 5.5 8.7) (end 5.7 8.5) (width 0.3) (layer "F.Cu") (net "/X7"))
 (segment (start 5.7 8.5) (end 6.1 8.3) (width 0.3) (layer "F.Cu") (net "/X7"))
 (segment (start 6.1 8.3) (end 12.7 7.7) (width 0.3) (layer "F.Cu") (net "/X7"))
 (segment (start 12.7 7.7) (end 13.3 7.1) (width 0.3) (layer "F.Cu") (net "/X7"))
 (segment (start 13.3 7.1) (end 33.9 8.3) (width 0.3) (layer "F.Cu") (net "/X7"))
 (segment (start 33.9 8.3) (end 34.3 8.5) (width 0.3) (layer "F.Cu") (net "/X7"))
 (segment (start 34.3 8.5) (end 34.7 8.9) (width 0.3) (layer "F.Cu") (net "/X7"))
 (segment (start 34.7 8.9) (end 34.7 12.3) (width 0.3) (layer "F.Cu") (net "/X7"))
 (segment (start 34.7 12.3) (end 34.7 14.3) (width 0.3) (layer "F.Cu") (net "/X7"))
 (segment (start 34.7 14.3) (end 34.7 14.9) (width 0.3) (layer "F.Cu") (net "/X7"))
 (segment (start 34.7 14.9) (end 34.9 15.3) (width 0.3) (layer "F.Cu") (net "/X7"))
 (segment (start 34.9 15.3) (end 35.7 16.5) (width 0.3) (layer "F.Cu") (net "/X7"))
 (segment (start 35.7 16.5) (end 36.04 17.16) (width 0.3) (layer "F.Cu") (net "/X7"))
 (segment (start 6.54 14.62) (end 7.3 14.9) (width 0.3) (layer "B.Cu") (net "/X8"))
 (segment (start 7.3 14.9) (end 14.5 14.9) (width 0.3) (layer "B.Cu") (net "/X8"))
 (segment (start 14.5 14.9) (end 16.1 15.7) (width 0.3) (layer "B.Cu") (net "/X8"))
 (segment (start 16.1 15.7) (end 22.1 17.9) (width 0.3) (layer "F.Cu") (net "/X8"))
 (segment (start 22.1 17.9) (end 28.1 17.7) (width 0.3) (layer "F.Cu") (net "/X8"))
 (segment (start 28.1 17.7) (end 28.3 17.5) (width 0.3) (layer "F.Cu") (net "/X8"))
 (segment (start 28.3 17.5) (end 32.7 17.3) (width 0.3) (layer "F.Cu") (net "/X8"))
 (segment (start 32.7 17.3) (end 33.5 17.16) (width 0.3) (layer "F.Cu") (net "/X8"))
 (segment (start 4 17.16) (end 4.7 17.5) (width 0.3) (layer "B.Cu") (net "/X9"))
 (segment (start 4.7 17.5) (end 5.9 18.3) (width 0.3) (layer "B.Cu") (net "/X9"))
 (segment (start 5.9 18.3) (end 6.3 18.5) (width 0.3) (layer "B.Cu") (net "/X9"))
 (segment (start 6.3 18.5) (end 13.3 18.5) (width 0.3) (layer "B.Cu") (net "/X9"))
 (segment (start 13.3 18.5) (end 16.9 19.3) (width 0.3) (layer "B.Cu") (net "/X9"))
 (segment (start 16.9 19.3) (end 17.5 19.3) (width 0.3) (layer "B.Cu") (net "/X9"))
 (segment (start 17.5 19.3) (end 18.5 18.5) (width 0.3) (layer "B.Cu") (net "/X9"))
 (segment (start 18.5 18.5) (end 19.5 18.5) (width 0.3) (layer "B.Cu") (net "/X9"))
 (segment (start 19.5 18.5) (end 21.5 18.9) (width 0.3) (layer "F.Cu") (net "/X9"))
 (segment (start 21.5 18.9) (end 28.5 18.5) (width 0.3) (layer "F.Cu") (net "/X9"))
 (segment (start 28.5 18.5) (end 33.1 15.9) (width 0.3) (layer "B.Cu") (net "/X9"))
 (segment (start 33.1 15.9) (end 33.9 15.9) (width 0.3) (layer "B.Cu") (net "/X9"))
 (segment (start 33.9 15.9) (end 34.3 15.7) (width 0.3) (layer "B.Cu") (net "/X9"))
 (segment (start 34.3 15.7) (end 35.3 14.9) (width 0.3) (layer "B.Cu") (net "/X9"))
 (segment (start 35.3 14.9) (end 36.04 14.62) (width 0.3) (layer "B.Cu") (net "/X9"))
 (segment (start 4 24.78) (end 4.7 24.7) (width 0.3) (layer "F.Cu") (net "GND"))
 (segment (start 4.7 24.7) (end 5.7 24.7) (width 0.3) (layer "F.Cu") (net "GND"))
 (segment (start 5.7 24.7) (end 6.54 24.78) (width 0.3) (layer "F.Cu") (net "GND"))
 (segment (start 4 24.78) (end 3.5 24.1) (width 0.3) (layer "F.Cu") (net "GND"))
 (segment (start 3.5 24.1) (end 2.7 22.7) (width 0.3) (layer "F.Cu") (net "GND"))
 (segment (start 2.7 22.7) (end 1.9 20.3) (width 0.3) (layer "F.Cu") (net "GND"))
 (segment (start 1.9 20.3) (end 1.9 16.5) (width 0.3) (layer "F.Cu") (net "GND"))
 (segment (start 1.9 16.5) (end 2.7 9.1) (width 0.3) (layer "F.Cu") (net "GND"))
 (segment (start 2.7 9.1) (end 3.5 8.3) (width 0.3) (layer "F.Cu") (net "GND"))
 (segment (start 3.5 8.3) (end 4.9 8.3) (width 0.3) (layer "F.Cu") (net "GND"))
 (segment (start 4.9 8.3) (end 5.3 7.9) (width 0.3) (layer "F.Cu") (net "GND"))
 (segment (start 5.3 7.9) (end 5.3 6.5) (width 0.3) (layer "F.Cu") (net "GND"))
 (segment (start 5.3 6.5) (end 6.1 5.7) (width 0.3) (layer "F.Cu") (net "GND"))
 (segment (start 6.1 5.7) (end 32.7 6.3) (width 0.3) (layer "F.Cu") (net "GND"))
 (segment (start 32.7 6.3) (end 33.5 7) (width 0.3) (layer "F.Cu") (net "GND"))
 (segment (start 33.5 7) (end 34.3 6.7) (width 0.3) (layer "F.Cu") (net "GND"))
 (segment (start 34.3 6.7) (end 35.3 6.7) (width 0.3) (layer "F.Cu") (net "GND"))
 (segment (start 35.3 6.7) (end 36.04 7) (width 0.3) (layer "F.Cu") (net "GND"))
 (via (at 15.3 9.3) (size 0.6) (drill 0.3) (layers "F.Cu" "B.Cu") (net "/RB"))
 (via (at 17.7 12.7) (size 0.6) (drill 0.3) (layers "F.Cu" "B.Cu") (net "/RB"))
 (via (at 10.5 21.5) (size 0.6) (drill 0.3) (layers "F.Cu" "B.Cu") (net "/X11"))
 (via (at 18.3 21.1) (size 0.6) (drill 0.3) (layers "F.Cu" "B.Cu") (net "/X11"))
 (via (at 17.5 13.7) (size 0.6) (drill 0.3) (layers "F.Cu" "B.Cu") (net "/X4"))
 (via (at 27.9 16.7) (size 0.6) (drill 0.3) (layers "F.Cu" "B.Cu") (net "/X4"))
 (via (at 17.1 18.3) (size 0.6) (drill 0.3) (layers "F.Cu" "B.Cu") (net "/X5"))
 (via (at 31.9 19.9) (size 0.6) (drill 0.3) (layers "F.Cu" "B.Cu") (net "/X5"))
 (via (at 21.7 14.3) (size 0.6) (drill 0.3) (layers "F.Cu" "B.Cu") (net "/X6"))
 (via (at 16.1 15.7) (size 0.6) (drill 0.3) (layers "F.Cu" "B.Cu") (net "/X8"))
 (via (at 19.5 18.5) (size 0.6) (drill 0.3) (layers "F.Cu" "B.Cu") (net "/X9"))
 (via (at 28.5 18.5) (size 0.6) (drill 0.3) (layers "F.Cu" "B.Cu") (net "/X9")))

